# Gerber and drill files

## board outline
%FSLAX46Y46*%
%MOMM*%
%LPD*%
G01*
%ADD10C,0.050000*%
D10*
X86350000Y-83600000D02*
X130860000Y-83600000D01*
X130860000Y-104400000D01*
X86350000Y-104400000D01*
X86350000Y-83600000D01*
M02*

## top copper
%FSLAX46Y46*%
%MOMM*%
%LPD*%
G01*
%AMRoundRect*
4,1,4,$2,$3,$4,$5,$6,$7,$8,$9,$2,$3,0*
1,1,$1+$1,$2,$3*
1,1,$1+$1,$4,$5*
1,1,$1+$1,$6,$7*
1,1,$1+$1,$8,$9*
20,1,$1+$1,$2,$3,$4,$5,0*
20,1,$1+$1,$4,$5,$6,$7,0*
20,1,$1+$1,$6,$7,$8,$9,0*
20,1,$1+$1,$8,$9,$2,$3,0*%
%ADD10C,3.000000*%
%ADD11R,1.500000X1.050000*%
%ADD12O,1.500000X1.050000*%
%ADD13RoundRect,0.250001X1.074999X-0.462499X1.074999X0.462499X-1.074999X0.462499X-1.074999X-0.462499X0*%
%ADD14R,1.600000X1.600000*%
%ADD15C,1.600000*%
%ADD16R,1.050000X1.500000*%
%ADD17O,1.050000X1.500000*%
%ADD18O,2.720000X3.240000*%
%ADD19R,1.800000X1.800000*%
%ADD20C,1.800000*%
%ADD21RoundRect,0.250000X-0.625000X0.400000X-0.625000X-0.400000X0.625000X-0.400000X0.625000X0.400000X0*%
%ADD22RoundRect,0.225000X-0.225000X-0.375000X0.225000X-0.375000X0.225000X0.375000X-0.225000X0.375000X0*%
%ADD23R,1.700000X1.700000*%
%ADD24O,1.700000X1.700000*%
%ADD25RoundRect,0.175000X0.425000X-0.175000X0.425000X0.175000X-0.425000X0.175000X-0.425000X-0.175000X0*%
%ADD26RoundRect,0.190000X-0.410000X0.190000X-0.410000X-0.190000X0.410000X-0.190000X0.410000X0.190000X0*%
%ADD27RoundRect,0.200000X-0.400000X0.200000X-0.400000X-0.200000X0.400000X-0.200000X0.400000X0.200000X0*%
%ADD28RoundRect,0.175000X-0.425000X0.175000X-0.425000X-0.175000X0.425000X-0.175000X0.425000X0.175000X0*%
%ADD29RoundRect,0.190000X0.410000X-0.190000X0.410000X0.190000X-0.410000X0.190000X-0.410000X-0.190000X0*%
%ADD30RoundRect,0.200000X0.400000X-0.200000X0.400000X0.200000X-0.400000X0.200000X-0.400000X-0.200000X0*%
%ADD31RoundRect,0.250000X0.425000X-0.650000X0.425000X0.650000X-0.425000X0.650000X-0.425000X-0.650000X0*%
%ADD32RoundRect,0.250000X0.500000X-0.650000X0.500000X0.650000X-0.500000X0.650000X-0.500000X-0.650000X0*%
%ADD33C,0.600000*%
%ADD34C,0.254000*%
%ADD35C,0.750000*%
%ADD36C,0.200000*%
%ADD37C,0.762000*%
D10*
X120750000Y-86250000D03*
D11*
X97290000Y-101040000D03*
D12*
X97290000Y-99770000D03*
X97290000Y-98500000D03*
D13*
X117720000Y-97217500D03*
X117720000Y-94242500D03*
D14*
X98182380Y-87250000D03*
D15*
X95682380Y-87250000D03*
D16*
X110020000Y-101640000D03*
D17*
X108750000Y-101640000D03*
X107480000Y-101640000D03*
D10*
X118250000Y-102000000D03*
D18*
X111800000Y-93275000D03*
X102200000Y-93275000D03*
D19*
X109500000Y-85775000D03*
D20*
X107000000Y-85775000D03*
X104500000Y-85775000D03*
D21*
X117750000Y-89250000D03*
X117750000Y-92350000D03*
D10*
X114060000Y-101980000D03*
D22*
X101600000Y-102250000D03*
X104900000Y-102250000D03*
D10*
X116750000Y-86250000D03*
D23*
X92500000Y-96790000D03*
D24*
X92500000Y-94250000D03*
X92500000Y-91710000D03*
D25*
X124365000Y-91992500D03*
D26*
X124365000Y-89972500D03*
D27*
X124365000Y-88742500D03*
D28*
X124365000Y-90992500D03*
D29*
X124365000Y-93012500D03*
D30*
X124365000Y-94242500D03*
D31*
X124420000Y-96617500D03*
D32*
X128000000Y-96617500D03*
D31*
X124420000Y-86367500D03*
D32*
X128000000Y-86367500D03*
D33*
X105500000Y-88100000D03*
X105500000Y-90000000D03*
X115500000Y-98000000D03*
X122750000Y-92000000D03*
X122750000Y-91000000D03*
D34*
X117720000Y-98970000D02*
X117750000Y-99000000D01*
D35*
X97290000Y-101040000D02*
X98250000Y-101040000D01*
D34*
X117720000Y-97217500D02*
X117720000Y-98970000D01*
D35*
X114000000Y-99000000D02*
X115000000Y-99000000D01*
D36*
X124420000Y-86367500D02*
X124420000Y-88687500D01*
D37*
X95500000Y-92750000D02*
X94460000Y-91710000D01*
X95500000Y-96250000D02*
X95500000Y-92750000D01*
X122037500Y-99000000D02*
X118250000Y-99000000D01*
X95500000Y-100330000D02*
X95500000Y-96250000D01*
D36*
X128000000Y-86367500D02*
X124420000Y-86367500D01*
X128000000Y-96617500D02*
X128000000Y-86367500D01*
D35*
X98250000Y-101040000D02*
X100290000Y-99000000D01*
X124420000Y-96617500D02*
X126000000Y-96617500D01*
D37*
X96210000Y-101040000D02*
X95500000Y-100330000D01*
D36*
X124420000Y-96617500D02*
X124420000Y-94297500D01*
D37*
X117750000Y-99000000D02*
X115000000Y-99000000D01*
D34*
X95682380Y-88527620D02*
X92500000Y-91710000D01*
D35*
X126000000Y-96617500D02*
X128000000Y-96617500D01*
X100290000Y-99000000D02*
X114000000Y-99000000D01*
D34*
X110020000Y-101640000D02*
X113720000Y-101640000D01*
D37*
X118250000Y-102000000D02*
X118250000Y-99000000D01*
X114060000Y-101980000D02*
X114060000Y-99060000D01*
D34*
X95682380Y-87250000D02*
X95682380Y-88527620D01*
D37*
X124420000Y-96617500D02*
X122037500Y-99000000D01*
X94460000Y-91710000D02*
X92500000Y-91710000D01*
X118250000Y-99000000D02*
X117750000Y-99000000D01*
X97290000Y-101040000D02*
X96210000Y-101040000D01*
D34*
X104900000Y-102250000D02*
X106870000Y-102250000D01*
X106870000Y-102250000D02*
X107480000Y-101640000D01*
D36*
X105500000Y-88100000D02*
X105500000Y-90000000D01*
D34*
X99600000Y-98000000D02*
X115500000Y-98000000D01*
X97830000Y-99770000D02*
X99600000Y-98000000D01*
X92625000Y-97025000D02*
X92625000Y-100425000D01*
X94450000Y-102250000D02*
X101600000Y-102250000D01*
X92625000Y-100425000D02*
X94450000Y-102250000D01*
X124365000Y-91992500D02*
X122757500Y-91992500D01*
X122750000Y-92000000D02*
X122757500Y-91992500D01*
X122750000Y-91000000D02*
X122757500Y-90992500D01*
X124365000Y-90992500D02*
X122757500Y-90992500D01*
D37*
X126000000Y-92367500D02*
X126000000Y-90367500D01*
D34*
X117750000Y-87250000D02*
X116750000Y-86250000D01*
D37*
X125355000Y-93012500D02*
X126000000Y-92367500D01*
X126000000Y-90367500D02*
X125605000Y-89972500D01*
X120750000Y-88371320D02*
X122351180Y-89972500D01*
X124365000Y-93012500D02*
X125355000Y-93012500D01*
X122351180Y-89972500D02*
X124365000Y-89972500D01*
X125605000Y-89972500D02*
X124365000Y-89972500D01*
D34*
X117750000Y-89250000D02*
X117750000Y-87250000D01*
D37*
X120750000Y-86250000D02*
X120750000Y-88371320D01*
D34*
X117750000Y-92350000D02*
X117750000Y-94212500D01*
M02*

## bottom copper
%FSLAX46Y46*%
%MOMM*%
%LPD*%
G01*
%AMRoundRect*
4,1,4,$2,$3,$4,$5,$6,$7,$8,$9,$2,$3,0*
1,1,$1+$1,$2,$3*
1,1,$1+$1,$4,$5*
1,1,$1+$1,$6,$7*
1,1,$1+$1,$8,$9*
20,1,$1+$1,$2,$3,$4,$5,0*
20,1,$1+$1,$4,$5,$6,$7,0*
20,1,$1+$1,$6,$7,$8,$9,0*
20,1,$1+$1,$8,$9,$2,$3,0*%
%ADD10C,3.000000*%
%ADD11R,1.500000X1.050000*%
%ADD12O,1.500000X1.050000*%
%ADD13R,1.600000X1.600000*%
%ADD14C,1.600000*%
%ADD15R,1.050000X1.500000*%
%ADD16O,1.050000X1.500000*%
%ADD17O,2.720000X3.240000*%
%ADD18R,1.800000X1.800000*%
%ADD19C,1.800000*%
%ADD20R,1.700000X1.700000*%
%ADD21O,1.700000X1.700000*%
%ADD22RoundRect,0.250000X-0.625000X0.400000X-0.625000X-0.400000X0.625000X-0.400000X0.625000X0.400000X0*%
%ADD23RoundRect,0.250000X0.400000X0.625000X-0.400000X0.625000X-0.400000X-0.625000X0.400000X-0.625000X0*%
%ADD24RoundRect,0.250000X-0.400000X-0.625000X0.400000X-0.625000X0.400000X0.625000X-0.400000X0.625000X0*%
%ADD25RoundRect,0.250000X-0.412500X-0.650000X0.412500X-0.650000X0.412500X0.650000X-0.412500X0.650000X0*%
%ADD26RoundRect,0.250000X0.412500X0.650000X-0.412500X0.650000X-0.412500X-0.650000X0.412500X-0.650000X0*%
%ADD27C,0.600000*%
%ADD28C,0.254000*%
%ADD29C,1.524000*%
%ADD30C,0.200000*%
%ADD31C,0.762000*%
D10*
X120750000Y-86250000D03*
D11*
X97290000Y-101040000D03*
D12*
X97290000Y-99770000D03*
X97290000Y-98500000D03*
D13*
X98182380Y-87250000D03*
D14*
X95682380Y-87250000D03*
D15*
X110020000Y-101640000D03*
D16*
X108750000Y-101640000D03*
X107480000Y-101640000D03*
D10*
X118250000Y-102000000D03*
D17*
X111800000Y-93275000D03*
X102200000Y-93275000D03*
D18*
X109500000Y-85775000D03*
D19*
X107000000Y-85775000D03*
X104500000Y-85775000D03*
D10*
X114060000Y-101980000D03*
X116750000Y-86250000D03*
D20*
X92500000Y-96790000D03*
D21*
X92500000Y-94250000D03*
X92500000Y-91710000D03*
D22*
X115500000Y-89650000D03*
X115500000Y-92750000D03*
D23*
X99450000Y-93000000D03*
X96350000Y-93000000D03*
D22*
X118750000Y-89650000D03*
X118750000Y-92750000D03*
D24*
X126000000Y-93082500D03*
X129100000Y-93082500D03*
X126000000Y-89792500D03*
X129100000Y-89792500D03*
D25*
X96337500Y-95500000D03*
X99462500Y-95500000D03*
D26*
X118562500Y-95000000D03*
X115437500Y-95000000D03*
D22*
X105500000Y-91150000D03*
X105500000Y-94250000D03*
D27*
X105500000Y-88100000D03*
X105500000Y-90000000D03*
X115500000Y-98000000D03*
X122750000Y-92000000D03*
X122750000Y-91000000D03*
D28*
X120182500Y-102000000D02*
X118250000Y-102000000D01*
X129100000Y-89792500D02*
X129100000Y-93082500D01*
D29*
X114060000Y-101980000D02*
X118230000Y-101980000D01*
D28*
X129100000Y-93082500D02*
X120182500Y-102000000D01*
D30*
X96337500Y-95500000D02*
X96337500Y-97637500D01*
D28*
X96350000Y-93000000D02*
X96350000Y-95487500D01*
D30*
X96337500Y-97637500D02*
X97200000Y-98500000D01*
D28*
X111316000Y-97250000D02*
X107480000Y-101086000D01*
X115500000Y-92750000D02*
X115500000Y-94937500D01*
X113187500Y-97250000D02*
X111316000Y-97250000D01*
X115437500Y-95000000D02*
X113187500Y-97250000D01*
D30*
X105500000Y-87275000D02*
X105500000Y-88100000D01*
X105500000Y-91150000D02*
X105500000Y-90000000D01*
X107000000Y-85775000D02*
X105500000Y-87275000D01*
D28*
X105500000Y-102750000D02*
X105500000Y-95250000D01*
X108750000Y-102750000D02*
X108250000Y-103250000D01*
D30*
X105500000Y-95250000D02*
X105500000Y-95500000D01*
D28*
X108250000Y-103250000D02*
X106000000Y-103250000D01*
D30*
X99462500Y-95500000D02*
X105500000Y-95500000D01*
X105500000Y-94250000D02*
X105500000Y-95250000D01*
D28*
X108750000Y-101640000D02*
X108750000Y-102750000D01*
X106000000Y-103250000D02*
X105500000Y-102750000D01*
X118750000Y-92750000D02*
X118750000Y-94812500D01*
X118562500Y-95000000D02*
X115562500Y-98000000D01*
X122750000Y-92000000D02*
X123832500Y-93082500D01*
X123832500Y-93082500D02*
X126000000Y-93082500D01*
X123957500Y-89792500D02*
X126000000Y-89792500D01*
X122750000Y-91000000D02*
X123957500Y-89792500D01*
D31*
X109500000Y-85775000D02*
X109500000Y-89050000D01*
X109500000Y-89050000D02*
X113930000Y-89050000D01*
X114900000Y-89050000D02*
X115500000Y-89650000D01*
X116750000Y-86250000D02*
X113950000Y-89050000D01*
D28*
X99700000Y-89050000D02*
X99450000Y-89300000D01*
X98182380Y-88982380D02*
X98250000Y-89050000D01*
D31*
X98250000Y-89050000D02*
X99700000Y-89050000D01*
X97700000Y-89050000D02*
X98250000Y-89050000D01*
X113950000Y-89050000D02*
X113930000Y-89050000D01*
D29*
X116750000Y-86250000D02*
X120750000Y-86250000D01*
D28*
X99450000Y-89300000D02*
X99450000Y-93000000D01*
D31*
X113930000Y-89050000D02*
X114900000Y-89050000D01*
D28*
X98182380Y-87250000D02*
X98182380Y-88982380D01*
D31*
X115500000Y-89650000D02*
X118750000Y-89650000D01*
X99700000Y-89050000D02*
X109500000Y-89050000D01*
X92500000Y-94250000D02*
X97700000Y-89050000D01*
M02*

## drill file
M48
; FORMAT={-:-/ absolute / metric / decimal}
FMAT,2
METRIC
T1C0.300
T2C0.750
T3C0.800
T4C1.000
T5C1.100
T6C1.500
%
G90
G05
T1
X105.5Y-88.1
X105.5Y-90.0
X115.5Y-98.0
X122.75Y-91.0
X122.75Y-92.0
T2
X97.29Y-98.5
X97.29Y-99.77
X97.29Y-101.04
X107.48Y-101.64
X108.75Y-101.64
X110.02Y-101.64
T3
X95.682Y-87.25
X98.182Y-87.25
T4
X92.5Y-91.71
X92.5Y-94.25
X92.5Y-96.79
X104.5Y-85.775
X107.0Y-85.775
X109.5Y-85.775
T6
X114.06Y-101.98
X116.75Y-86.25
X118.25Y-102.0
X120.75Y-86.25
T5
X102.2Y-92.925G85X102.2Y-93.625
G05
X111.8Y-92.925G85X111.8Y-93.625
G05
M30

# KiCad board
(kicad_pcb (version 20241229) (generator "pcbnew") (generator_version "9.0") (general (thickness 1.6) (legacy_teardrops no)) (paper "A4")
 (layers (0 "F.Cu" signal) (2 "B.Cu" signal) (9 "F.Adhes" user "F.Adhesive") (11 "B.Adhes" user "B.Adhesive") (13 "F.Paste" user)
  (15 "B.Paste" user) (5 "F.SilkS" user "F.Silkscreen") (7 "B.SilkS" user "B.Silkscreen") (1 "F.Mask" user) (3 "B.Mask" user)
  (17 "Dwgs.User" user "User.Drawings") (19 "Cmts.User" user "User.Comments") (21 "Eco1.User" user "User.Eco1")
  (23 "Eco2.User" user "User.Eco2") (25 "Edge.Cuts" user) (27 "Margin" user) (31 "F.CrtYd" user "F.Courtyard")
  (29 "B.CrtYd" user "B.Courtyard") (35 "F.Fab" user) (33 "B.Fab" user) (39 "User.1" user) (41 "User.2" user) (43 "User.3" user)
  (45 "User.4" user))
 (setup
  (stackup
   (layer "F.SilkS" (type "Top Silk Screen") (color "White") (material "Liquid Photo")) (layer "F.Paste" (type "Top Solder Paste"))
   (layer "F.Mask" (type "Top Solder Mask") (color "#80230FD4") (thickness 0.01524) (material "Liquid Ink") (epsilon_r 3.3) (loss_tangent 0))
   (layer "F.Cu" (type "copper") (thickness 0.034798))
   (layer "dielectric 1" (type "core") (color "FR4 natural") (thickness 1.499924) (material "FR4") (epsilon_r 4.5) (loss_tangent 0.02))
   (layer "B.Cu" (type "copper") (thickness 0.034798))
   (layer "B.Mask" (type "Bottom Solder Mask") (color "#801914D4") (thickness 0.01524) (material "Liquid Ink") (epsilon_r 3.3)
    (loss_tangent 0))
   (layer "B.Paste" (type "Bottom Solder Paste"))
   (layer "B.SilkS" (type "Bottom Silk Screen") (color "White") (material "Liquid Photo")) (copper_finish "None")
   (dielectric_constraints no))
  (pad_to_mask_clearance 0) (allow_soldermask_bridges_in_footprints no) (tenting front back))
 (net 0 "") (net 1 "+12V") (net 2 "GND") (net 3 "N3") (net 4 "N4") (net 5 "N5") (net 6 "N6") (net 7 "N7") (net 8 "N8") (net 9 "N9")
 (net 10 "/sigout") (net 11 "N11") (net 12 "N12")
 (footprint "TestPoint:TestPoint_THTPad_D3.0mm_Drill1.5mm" (layer "F.Cu") (at 120.75 86.25)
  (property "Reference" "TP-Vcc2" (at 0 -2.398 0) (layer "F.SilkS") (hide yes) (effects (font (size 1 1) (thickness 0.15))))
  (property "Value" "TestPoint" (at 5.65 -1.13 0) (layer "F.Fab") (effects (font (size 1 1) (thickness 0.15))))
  (pad "1" thru_hole circle (at 0 0) (size 3 3) (drill 1.5) (layers "*.Cu" "*.Mask") (remove_unused_layers no) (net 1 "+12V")))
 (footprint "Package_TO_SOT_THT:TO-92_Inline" (layer "F.Cu") (at 97.29 101.04 90)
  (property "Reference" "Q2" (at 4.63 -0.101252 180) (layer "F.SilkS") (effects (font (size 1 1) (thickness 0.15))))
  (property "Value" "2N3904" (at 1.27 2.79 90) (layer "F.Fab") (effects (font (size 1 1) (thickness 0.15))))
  (pad "1" thru_hole rect (at 0 0 90) (size 1.05 1.5) (drill 0.75) (layers "*.Cu" "*.Mask") (remove_unused_layers no) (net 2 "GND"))
  (pad "2" thru_hole oval (at 1.27 0 90) (size 1.05 1.5) (drill 0.75) (layers "*.Cu" "*.Mask") (remove_unused_layers no) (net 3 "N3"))
  (pad "3" thru_hole oval (at 2.54 0 90) (size 1.05 1.5) (drill 0.75) (layers "*.Cu" "*.Mask") (remove_unused_layers no) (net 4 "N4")))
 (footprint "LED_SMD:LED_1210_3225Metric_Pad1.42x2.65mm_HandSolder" (layer "F.Cu") (at 117.72 95.73 90)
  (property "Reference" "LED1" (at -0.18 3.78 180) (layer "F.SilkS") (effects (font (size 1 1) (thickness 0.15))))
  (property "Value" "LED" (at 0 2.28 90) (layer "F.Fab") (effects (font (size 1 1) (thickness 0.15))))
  (pad "1" smd roundrect (at -1.4875 0 90) (size 1.425 2.65) (layers "F.Cu" "F.Mask" "F.Paste") (roundrect_rratio 0.175439) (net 2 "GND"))
  (pad "2" smd roundrect (at 1.4875 0 90) (size 1.425 2.65) (layers "F.Cu" "F.Mask" "F.Paste") (roundrect_rratio 0.175439) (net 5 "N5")))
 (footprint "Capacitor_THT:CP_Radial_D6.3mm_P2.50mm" (layer "F.Cu") (at 98.18238 87.25 180)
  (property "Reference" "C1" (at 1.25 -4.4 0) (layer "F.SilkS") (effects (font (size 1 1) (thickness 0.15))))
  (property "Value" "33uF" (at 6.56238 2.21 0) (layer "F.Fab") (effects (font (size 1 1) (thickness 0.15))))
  (pad "1" thru_hole rect (at 0 0 180) (size 1.6 1.6) (drill 0.8) (layers "*.Cu" "*.Mask") (remove_unused_layers no) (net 1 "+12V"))
  (pad "2" thru_hole circle (at 2.5 0 180) (size 1.6 1.6) (drill 0.8) (layers "*.Cu" "*.Mask") (remove_unused_layers no) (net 2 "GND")))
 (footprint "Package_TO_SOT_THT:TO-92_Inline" (layer "F.Cu") (at 110.02 101.64 180)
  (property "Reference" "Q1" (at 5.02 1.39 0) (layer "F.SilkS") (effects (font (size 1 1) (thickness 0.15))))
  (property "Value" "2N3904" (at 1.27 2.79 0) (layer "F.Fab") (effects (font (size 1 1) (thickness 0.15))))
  (pad "1" thru_hole rect (at 0 0 180) (size 1.05 1.5) (drill 0.75) (layers "*.Cu" "*.Mask") (remove_unused_layers no) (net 2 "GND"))
  (pad "2" thru_hole oval (at 1.27 0 180) (size 1.05 1.5) (drill 0.75) (layers "*.Cu" "*.Mask") (remove_unused_layers no) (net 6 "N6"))
  (pad "3" thru_hole oval (at 2.54 0 180) (size 1.05 1.5) (drill 0.75) (layers "*.Cu" "*.Mask") (remove_unused_layers no) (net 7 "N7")))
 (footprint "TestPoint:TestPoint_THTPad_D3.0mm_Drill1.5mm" (layer "F.Cu") (at 118.25 102)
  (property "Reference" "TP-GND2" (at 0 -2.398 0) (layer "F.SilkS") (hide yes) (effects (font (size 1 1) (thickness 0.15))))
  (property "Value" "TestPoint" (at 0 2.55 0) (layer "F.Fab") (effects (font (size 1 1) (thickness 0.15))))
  (pad "1" thru_hole circle (at 0 0) (size 3 3) (drill 1.5) (layers "*.Cu" "*.Mask") (remove_unused_layers no) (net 2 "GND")))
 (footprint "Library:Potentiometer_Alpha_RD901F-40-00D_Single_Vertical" (layer "F.Cu") (at 109.5 85.775 -90)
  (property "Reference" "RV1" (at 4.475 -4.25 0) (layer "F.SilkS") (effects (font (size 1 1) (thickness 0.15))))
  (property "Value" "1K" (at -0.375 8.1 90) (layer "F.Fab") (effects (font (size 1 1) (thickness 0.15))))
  (pad "" thru_hole oval (at 7.5 -2.3) (size 2.72 3.24) (drill oval 1.1 1.8) (layers "*.Cu" "*.Mask") (remove_unused_layers no))
  (pad "" thru_hole oval (at 7.5 7.3) (size 2.72 3.24) (drill oval 1.1 1.8) (layers "*.Cu" "*.Mask") (remove_unused_layers no))
  (pad "1" thru_hole rect (at 0 0) (size 1.8 1.8) (drill 1) (layers "*.Cu" "*.Mask") (remove_unused_layers no) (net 1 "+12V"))
  (pad "2" thru_hole circle (at 0 2.5) (size 1.8 1.8) (drill 1) (layers "*.Cu" "*.Mask") (remove_unused_layers no) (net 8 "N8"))
  (pad "3" thru_hole circle (at 0 5) (size 1.8 1.8) (drill 1) (layers "*.Cu" "*.Mask") (remove_unused_layers no) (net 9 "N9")))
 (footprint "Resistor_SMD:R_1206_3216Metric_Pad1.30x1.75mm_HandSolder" (layer "F.Cu") (at 117.75 90.8 -90)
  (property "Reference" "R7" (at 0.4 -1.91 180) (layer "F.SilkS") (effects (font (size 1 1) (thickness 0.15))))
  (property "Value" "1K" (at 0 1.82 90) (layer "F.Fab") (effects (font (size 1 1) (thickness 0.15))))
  (pad "1" smd roundrect (at -1.55 0 270) (size 1.3 1.75) (layers "F.Cu" "F.Mask" "F.Paste") (roundrect_rratio 0.192308) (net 1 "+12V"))
  (pad "2" smd roundrect (at 1.55 0 270) (size 1.3 1.75) (layers "F.Cu" "F.Mask" "F.Paste") (roundrect_rratio 0.192308) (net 5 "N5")))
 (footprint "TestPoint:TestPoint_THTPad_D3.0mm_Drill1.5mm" (layer "F.Cu") (at 114.06 101.98)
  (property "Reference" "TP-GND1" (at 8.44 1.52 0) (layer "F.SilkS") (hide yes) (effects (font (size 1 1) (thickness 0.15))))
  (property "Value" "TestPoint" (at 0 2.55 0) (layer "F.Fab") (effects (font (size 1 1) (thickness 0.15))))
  (pad "1" thru_hole circle (at 0 0) (size 3 3) (drill 1.5) (layers "*.Cu" "*.Mask") (remove_unused_layers no) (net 2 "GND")))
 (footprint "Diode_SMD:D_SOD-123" (layer "F.Cu") (at 103.25 102.25)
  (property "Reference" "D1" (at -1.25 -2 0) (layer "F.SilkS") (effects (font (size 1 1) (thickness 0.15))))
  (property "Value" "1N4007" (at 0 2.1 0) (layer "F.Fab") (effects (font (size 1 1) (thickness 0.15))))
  (pad "1" smd roundrect (at -1.65 0) (size 0.9 1.2) (layers "F.Cu" "F.Mask" "F.Paste") (roundrect_rratio 0.25) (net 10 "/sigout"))
  (pad "2" smd roundrect (at 1.65 0) (size 0.9 1.2) (layers "F.Cu" "F.Mask" "F.Paste") (roundrect_rratio 0.25) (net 7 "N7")))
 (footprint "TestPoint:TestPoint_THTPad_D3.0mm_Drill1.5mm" (layer "F.Cu") (at 116.75 86.25)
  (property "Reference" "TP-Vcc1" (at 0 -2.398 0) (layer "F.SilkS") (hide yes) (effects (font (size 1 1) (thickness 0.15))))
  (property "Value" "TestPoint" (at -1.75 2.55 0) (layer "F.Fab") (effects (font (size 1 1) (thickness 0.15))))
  (pad "1" thru_hole circle (at 0 0) (size 3 3) (drill 1.5) (layers "*.Cu" "*.Mask") (remove_unused_layers no) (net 1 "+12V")))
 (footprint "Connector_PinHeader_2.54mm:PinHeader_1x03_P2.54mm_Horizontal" (layer "F.Cu") (at 92.5 96.79 180)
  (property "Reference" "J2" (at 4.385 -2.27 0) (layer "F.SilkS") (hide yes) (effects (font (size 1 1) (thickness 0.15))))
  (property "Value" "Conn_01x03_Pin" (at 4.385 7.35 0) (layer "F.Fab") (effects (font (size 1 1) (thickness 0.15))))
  (pad "1" thru_hole rect (at 0 0 180) (size 1.7 1.7) (drill 1) (layers "*.Cu" "*.Mask") (remove_unused_layers no) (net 10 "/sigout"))
  (pad "2" thru_hole oval (at 0 2.54 180) (size 1.7 1.7) (drill 1) (layers "*.Cu" "*.Mask") (remove_unused_layers no) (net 1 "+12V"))
  (pad "3" thru_hole oval (at 0 5.08 180) (size 1.7 1.7) (drill 1) (layers "*.Cu" "*.Mask") (remove_unused_layers no) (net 2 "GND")))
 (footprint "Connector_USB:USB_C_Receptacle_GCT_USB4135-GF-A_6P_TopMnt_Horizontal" (layer "F.Cu") (at 127.3975 91.4925 90)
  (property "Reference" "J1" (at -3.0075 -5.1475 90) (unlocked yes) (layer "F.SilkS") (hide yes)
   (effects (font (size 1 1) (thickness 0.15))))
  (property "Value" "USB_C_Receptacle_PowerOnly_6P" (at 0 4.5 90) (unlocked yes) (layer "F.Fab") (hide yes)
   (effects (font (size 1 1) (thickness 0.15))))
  (pad "A5" smd roundrect (at -0.5 -3.0325 90) (size 0.7 1.2) (layers "F.Cu" "F.Mask" "F.Paste") (roundrect_rratio 0.25) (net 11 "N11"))
  (pad "A9" smd roundrect (at 1.52 -3.0325 270) (size 0.76 1.2) (layers "F.Cu" "F.Mask" "F.Paste") (roundrect_rratio 0.25) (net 1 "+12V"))
  (pad "A12" smd roundrect (at 2.75 -3.0325 270) (size 0.8 1.2) (layers "F.Cu" "F.Mask" "F.Paste") (roundrect_rratio 0.25) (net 2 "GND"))
  (pad "B5" smd roundrect (at 0.5 -3.0325 270) (size 0.7 1.2) (layers "F.Cu" "F.Mask" "F.Paste") (roundrect_rratio 0.25) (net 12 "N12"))
  (pad "B9" smd roundrect (at -1.52 -3.0325 90) (size 0.76 1.2) (layers "F.Cu" "F.Mask" "F.Paste") (roundrect_rratio 0.25) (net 1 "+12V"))
  (pad "B12" smd roundrect (at -2.75 -3.0325 90) (size 0.8 1.2) (layers "F.Cu" "F.Mask" "F.Paste") (roundrect_rratio 0.25) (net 2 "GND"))
  (pad "S1" smd roundrect (at -5.125 -2.9775 90) (size 1.8 1.35) (layers "F.Cu" "F.Mask" "F.Paste") (roundrect_rratio 0.1851851852)
   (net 2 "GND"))
  (pad "S1" smd roundrect (at -5.125 0.6025 90) (size 1.8 1.5) (layers "F.Cu" "F.Mask" "F.Paste") (roundrect_rratio 0.1666666667)
   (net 2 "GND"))
  (pad "S1" smd roundrect (at 5.125 -2.9775 90) (size 1.8 1.35) (layers "F.Cu" "F.Mask" "F.Paste") (roundrect_rratio 0.1851851852)
   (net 2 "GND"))
  (pad "S1" smd roundrect (at 5.125 0.6025 90) (size 1.8 1.5) (layers "F.Cu" "F.Mask" "F.Paste") (roundrect_rratio 0.1666666667)
   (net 2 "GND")))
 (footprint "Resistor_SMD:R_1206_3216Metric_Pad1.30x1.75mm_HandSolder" (layer "B.Cu") (at 115.5 91.2 -90)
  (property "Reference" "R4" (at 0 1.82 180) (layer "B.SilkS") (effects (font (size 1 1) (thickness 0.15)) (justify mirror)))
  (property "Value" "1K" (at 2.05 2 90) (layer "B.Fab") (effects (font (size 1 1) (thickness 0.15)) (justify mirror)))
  (pad "1" smd roundrect (at -1.55 0 270) (size 1.3 1.75) (layers "B.Cu" "B.Mask" "B.Paste") (roundrect_rratio 0.192308) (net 1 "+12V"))
  (pad "2" smd roundrect (at 1.55 0 270) (size 1.3 1.75) (layers "B.Cu" "B.Mask" "B.Paste") (roundrect_rratio 0.192308) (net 7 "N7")))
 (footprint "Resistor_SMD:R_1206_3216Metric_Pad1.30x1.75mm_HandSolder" (layer "B.Cu") (at 97.9 93 180)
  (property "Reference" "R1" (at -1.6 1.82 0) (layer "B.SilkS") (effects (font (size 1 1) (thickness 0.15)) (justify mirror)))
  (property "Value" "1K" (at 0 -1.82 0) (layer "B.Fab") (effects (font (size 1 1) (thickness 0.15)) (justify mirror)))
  (pad "1" smd roundrect (at -1.55 0 180) (size 1.3 1.75) (layers "B.Cu" "B.Mask" "B.Paste") (roundrect_rratio 0.192308) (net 1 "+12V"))
  (pad "2" smd roundrect (at 1.55 0 180) (size 1.3 1.75) (layers "B.Cu" "B.Mask" "B.Paste") (roundrect_rratio 0.192308) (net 4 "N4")))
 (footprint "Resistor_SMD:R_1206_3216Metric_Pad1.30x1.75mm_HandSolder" (layer "B.Cu") (at 118.75 91.2 -90)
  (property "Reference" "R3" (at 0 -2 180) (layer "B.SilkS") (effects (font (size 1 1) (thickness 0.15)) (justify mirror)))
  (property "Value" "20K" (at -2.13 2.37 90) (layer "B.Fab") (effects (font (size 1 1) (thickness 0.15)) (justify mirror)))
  (pad "1" smd roundrect (at -1.55 0 270) (size 1.3 1.75) (layers "B.Cu" "B.Mask" "B.Paste") (roundrect_rratio 0.192308) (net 1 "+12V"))
  (pad "2" smd roundrect (at 1.55 0 270) (size 1.3 1.75) (layers "B.Cu" "B.Mask" "B.Paste") (roundrect_rratio 0.192308) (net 3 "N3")))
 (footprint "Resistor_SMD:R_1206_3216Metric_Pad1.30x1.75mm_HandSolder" (layer "B.Cu") (at 127.55 93.0825)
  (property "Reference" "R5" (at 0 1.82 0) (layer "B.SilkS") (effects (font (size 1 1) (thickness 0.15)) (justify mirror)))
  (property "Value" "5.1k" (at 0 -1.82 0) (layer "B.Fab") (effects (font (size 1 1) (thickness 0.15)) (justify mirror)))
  (pad "1" smd roundrect (at -1.55 0) (size 1.3 1.75) (layers "B.Cu" "B.Mask" "B.Paste") (roundrect_rratio 0.192308) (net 11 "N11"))
  (pad "2" smd roundrect (at 1.55 0) (size 1.3 1.75) (layers "B.Cu" "B.Mask" "B.Paste") (roundrect_rratio 0.192308) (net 2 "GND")))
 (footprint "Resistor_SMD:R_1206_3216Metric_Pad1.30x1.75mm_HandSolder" (layer "B.Cu") (at 127.55 89.7925)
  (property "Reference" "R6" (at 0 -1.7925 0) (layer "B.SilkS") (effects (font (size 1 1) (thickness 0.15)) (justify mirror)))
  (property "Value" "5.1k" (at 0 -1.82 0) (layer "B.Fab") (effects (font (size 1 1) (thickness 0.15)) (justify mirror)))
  (pad "1" smd roundrect (at -1.55 0) (size 1.3 1.75) (layers "B.Cu" "B.Mask" "B.Paste") (roundrect_rratio 0.192308) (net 12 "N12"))
  (pad "2" smd roundrect (at 1.55 0) (size 1.3 1.75) (layers "B.Cu" "B.Mask" "B.Paste") (roundrect_rratio 0.192308) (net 2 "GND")))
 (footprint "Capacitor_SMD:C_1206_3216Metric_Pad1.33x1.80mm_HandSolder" (layer "B.Cu") (at 97.9 95.5)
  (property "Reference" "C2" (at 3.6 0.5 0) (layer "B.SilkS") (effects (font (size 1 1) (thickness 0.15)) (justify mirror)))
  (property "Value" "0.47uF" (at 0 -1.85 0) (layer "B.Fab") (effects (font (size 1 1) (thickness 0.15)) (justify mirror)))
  (pad "1" smd roundrect (at -1.5625 0) (size 1.325 1.8) (layers "B.Cu" "B.Mask" "B.Paste") (roundrect_rratio 0.188679) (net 4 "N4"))
  (pad "2" smd roundrect (at 1.5625 0) (size 1.325 1.8) (layers "B.Cu" "B.Mask" "B.Paste") (roundrect_rratio 0.188679) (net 6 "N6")))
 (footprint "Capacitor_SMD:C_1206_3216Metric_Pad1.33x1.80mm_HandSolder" (layer "B.Cu") (at 117 95 180)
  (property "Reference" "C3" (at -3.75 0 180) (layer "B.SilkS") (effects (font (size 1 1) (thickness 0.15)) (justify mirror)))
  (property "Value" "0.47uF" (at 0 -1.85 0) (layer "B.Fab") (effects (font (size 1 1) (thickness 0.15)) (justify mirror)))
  (pad "1" smd roundrect (at -1.5625 0 180) (size 1.325 1.8) (layers "B.Cu" "B.Mask" "B.Paste") (roundrect_rratio 0.188679) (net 3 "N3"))
  (pad "2" smd roundrect (at 1.5625 0 180) (size 1.325 1.8) (layers "B.Cu" "B.Mask" "B.Paste") (roundrect_rratio 0.188679) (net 7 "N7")))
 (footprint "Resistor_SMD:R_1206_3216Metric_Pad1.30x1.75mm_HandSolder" (layer "B.Cu") (at 105.5 92.7 -90)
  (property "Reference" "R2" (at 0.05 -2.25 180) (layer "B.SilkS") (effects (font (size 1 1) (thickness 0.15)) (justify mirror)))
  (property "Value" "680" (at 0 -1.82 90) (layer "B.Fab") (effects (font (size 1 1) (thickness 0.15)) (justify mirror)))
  (pad "1" smd roundrect (at -1.55 0 270) (size 1.3 1.75) (layers "B.Cu" "B.Mask" "B.Paste") (roundrect_rratio 0.192308) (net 8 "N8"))
  (pad "2" smd roundrect (at 1.55 0 270) (size 1.3 1.75) (layers "B.Cu" "B.Mask" "B.Paste") (roundrect_rratio 0.192308) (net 6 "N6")))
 (gr_rect (start 86.35 83.6) (end 130.86 104.4) (stroke (width 0.05) (type default)) (fill no) (layer "Edge.Cuts"))
 (segment (start 117.72 98.97) (end 117.75 99) (width 0.254) (layer "F.Cu") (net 2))
 (segment (start 97.29 101.04) (end 98.25 101.04) (width 0.75) (layer "F.Cu") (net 2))
 (segment (start 117.72 97.2175) (end 117.72 98.97) (width 0.254) (layer "F.Cu") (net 2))
 (segment (start 114 99) (end 115 99) (width 0.75) (layer "F.Cu") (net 2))
 (segment (start 124.42 86.3675) (end 124.42 88.6875) (width 0.2) (layer "F.Cu") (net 2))
 (segment (start 95.5 92.75) (end 94.46 91.71) (width 0.762) (layer "F.Cu") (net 2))
 (segment (start 95.5 96.25) (end 95.5 92.75) (width 0.762) (layer "F.Cu") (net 2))
 (segment (start 122.0375 99) (end 118.25 99) (width 0.762) (layer "F.Cu") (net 2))
 (segment (start 95.5 100.33) (end 95.5 96.25) (width 0.762) (layer "F.Cu") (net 2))
 (segment (start 128 86.3675) (end 124.42 86.3675) (width 0.2) (layer "F.Cu") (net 2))
 (segment (start 128 96.6175) (end 128 86.3675) (width 0.2) (layer "F.Cu") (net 2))
 (segment (start 98.25 101.04) (end 100.29 99) (width 0.75) (layer "F.Cu") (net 2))
 (segment (start 124.42 96.6175) (end 126 96.6175) (width 0.75) (layer "F.Cu") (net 2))
 (segment (start 96.21 101.04) (end 95.5 100.33) (width 0.762) (layer "F.Cu") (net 2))
 (segment (start 124.42 96.6175) (end 124.42 94.2975) (width 0.2) (layer "F.Cu") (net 2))
 (segment (start 117.75 99) (end 115 99) (width 0.762) (layer "F.Cu") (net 2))
 (segment (start 95.68238 88.52762) (end 92.5 91.71) (width 0.254) (layer "F.Cu") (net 2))
 (segment (start 126 96.6175) (end 128 96.6175) (width 0.75) (layer "F.Cu") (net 2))
 (segment (start 100.29 99) (end 114 99) (width 0.75) (layer "F.Cu") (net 2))
 (segment (start 110.02 101.64) (end 113.72 101.64) (width 0.254) (layer "F.Cu") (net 2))
 (segment (start 118.25 102) (end 118.25 99) (width 0.762) (layer "F.Cu") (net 2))
 (segment (start 114.06 101.98) (end 114.06 99.06) (width 0.762) (layer "F.Cu") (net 2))
 (segment (start 95.68238 87.25) (end 95.68238 88.52762) (width 0.254) (layer "F.Cu") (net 2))
 (segment (start 124.42 96.6175) (end 122.0375 99) (width 0.762) (layer "F.Cu") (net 2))
 (segment (start 94.46 91.71) (end 92.5 91.71) (width 0.762) (layer "F.Cu") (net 2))
 (segment (start 118.25 99) (end 117.75 99) (width 0.762) (layer "F.Cu") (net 2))
 (segment (start 97.29 101.04) (end 96.21 101.04) (width 0.762) (layer "F.Cu") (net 2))
 (segment (start 120.1825 102) (end 118.25 102) (width 0.254) (layer "B.Cu") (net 2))
 (segment (start 129.1 89.7925) (end 129.1 93.0825) (width 0.254) (layer "B.Cu") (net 2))
 (segment (start 114.06 101.98) (end 118.23 101.98) (width 1.524) (layer "B.Cu") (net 2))
 (segment (start 129.1 93.0825) (end 120.1825 102) (width 0.254) (layer "B.Cu") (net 2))
 (segment (start 96.3375 95.5) (end 96.3375 97.6375) (width 0.2) (layer "B.Cu") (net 4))
 (segment (start 96.35 93) (end 96.35 95.4875) (width 0.254) (layer "B.Cu") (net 4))
 (segment (start 96.3375 97.6375) (end 97.2 98.5) (width 0.2) (layer "B.Cu") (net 4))
 (segment (start 104.9 102.25) (end 106.87 102.25) (width 0.254) (layer "F.Cu") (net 7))
 (segment (start 106.87 102.25) (end 107.48 101.64) (width 0.254) (layer "F.Cu") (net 7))
 (segment (start 111.316 97.25) (end 107.48 101.086) (width 0.254) (layer "B.Cu") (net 7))
 (segment (start 115.5 92.75) (end 115.5 94.9375) (width 0.254) (layer "B.Cu") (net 7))
 (segment (start 113.1875 97.25) (end 111.316 97.25) (width 0.254) (layer "B.Cu") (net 7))
 (segment (start 115.4375 95) (end 113.1875 97.25) (width 0.254) (layer "B.Cu") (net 7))
 (segment (start 105.5 88.1) (end 105.5 90) (width 0.2) (layer "F.Cu") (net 8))
 (via (at 105.5 88.1) (size 0.6) (drill 0.3) (layers "F.Cu" "B.Cu") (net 8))
 (via (at 105.5 90) (size 0.6) (drill 0.3) (layers "F.Cu" "B.Cu") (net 8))
 (segment (start 105.5 87.275) (end 105.5 88.1) (width 0.2) (layer "B.Cu") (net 8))
 (segment (start 105.5 91.15) (end 105.5 90) (width 0.2) (layer "B.Cu") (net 8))
 (segment (start 107 85.775) (end 105.5 87.275) (width 0.2) (layer "B.Cu") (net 8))
 (segment (start 105.5 102.75) (end 105.5 95.25) (width 0.254) (layer "B.Cu") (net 6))
 (segment (start 108.75 102.75) (end 108.25 103.25) (width 0.254) (layer "B.Cu") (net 6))
 (segment (start 105.5 95.25) (end 105.5 95.5) (width 0.2) (layer "B.Cu") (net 6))
 (segment (start 108.25 103.25) (end 106 103.25) (width 0.254) (layer "B.Cu") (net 6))
 (segment (start 99.4625 95.5) (end 105.5 95.5) (width 0.2) (layer "B.Cu") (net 6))
 (segment (start 105.5 94.25) (end 105.5 95.25) (width 0.2) (layer "B.Cu") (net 6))
 (segment (start 108.75 101.64) (end 108.75 102.75) (width 0.254) (layer "B.Cu") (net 6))
 (segment (start 106 103.25) (end 105.5 102.75) (width 0.254) (layer "B.Cu") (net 6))
 (segment (start 99.6 98) (end 115.5 98) (width 0.254) (layer "F.Cu") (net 3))
 (segment (start 97.83 99.77) (end 99.6 98) (width 0.254) (layer "F.Cu") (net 3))
 (via (at 115.5 98) (size 0.6) (drill 0.3) (layers "F.Cu" "B.Cu") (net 3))
 (segment (start 118.75 92.75) (end 118.75 94.8125) (width 0.254) (layer "B.Cu") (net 3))
 (segment (start 118.5625 95) (end 115.5625 98) (width 0.254) (layer "B.Cu") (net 3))
 (segment (start 92.625 97.025) (end 92.625 100.425) (width 0.254) (layer "F.Cu") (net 10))
 (segment (start 94.45 102.25) (end 101.6 102.25) (width 0.254) (layer "F.Cu") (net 10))
 (segment (start 92.625 100.425) (end 94.45 102.25) (width 0.254) (layer "F.Cu") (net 10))
 (segment (start 124.365 91.9925) (end 122.7575 91.9925) (width 0.254) (layer "F.Cu") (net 11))
 (segment (start 122.75 92) (end 122.7575 91.9925) (width 0.254) (layer "F.Cu") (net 11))
 (via (at 122.75 92) (size 0.6) (drill 0.3) (layers "F.Cu" "B.Cu") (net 11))
 (segment (start 122.75 92) (end 123.8325 93.0825) (width 0.254) (layer "B.Cu") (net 11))
 (segment (start 123.8325 93.0825) (end 126 93.0825) (width 0.254) (layer "B.Cu") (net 11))
 (segment (start 122.75 91) (end 122.7575 90.9925) (width 0.254) (layer "F.Cu") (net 12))
 (segment (start 124.365 90.9925) (end 122.7575 90.9925) (width 0.254) (layer "F.Cu") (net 12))
 (via (at 122.75 91) (size 0.6) (drill 0.3) (layers "F.Cu" "B.Cu") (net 12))
 (segment (start 123.9575 89.7925) (end 126 89.7925) (width 0.254) (layer "B.Cu") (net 12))
 (segment (start 122.75 91) (end 123.9575 89.7925) (width 0.254) (layer "B.Cu") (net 12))
 (segment (start 126 92.3675) (end 126 90.3675) (width 0.762) (layer "F.Cu") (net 1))
 (segment (start 117.75 87.25) (end 116.75 86.25) (width 0.254) (layer "F.Cu") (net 1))
 (segment (start 125.355 93.0125) (end 126 92.3675) (width 0.762) (layer "F.Cu") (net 1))
 (segment (start 126 90.3675) (end 125.605 89.9725) (width 0.762) (layer "F.Cu") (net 1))
 (segment (start 120.75 88.37132) (end 122.35118 89.9725) (width 0.762) (layer "F.Cu") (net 1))
 (segment (start 124.365 93.0125) (end 125.355 93.0125) (width 0.762) (layer "F.Cu") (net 1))
 (segment (start 122.35118 89.9725) (end 124.365 89.9725) (width 0.762) (layer "F.Cu") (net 1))
 (segment (start 125.605 89.9725) (end 124.365 89.9725) (width 0.762) (layer "F.Cu") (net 1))
 (segment (start 117.75 89.25) (end 117.75 87.25) (width 0.254) (layer "F.Cu") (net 1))
 (segment (start 120.75 86.25) (end 120.75 88.37132) (width 0.762) (layer "F.Cu") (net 1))
 (segment (start 109.5 85.775) (end 109.5 89.05) (width 0.762) (layer "B.Cu") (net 1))
 (segment (start 109.5 89.05) (end 113.93 89.05) (width 0.762) (layer "B.Cu") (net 1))
 (segment (start 114.9 89.05) (end 115.5 89.65) (width 0.762) (layer "B.Cu") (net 1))
 (segment (start 116.75 86.25) (end 113.95 89.05) (width 0.762) (layer "B.Cu") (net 1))
 (segment (start 99.7 89.05) (end 99.45 89.3) (width 0.254) (layer "B.Cu") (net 1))
 (segment (start 98.18238 88.98238) (end 98.25 89.05) (width 0.254) (layer "B.Cu") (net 1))
 (segment (start 98.25 89.05) (end 99.7 89.05) (width 0.762) (layer "B.Cu") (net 1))
 (segment (start 97.7 89.05) (end 98.25 89.05) (width 0.762) (layer "B.Cu") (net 1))
 (segment (start 113.95 89.05) (end 113.93 89.05) (width 0.762) (layer "B.Cu") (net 1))
 (segment (start 116.75 86.25) (end 120.75 86.25) (width 1.524) (layer "B.Cu") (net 1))
 (segment (start 99.45 89.3) (end 99.45 93) (width 0.254) (layer "B.Cu") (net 1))
 (segment (start 113.93 89.05) (end 114.9 89.05) (width 0.762) (layer "B.Cu") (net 1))
 (segment (start 98.18238 87.25) (end 98.18238 88.98238) (width 0.254) (layer "B.Cu") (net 1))
 (segment (start 115.5 89.65) (end 118.75 89.65) (width 0.762) (layer "B.Cu") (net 1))
 (segment (start 99.7 89.05) (end 109.5 89.05) (width 0.762) (layer "B.Cu") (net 1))
 (segment (start 92.5 94.25) (end 97.7 89.05) (width 0.762) (layer "B.Cu") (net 1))
 (segment (start 117.75 92.35) (end 117.75 94.2125) (width 0.254) (layer "F.Cu") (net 5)))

